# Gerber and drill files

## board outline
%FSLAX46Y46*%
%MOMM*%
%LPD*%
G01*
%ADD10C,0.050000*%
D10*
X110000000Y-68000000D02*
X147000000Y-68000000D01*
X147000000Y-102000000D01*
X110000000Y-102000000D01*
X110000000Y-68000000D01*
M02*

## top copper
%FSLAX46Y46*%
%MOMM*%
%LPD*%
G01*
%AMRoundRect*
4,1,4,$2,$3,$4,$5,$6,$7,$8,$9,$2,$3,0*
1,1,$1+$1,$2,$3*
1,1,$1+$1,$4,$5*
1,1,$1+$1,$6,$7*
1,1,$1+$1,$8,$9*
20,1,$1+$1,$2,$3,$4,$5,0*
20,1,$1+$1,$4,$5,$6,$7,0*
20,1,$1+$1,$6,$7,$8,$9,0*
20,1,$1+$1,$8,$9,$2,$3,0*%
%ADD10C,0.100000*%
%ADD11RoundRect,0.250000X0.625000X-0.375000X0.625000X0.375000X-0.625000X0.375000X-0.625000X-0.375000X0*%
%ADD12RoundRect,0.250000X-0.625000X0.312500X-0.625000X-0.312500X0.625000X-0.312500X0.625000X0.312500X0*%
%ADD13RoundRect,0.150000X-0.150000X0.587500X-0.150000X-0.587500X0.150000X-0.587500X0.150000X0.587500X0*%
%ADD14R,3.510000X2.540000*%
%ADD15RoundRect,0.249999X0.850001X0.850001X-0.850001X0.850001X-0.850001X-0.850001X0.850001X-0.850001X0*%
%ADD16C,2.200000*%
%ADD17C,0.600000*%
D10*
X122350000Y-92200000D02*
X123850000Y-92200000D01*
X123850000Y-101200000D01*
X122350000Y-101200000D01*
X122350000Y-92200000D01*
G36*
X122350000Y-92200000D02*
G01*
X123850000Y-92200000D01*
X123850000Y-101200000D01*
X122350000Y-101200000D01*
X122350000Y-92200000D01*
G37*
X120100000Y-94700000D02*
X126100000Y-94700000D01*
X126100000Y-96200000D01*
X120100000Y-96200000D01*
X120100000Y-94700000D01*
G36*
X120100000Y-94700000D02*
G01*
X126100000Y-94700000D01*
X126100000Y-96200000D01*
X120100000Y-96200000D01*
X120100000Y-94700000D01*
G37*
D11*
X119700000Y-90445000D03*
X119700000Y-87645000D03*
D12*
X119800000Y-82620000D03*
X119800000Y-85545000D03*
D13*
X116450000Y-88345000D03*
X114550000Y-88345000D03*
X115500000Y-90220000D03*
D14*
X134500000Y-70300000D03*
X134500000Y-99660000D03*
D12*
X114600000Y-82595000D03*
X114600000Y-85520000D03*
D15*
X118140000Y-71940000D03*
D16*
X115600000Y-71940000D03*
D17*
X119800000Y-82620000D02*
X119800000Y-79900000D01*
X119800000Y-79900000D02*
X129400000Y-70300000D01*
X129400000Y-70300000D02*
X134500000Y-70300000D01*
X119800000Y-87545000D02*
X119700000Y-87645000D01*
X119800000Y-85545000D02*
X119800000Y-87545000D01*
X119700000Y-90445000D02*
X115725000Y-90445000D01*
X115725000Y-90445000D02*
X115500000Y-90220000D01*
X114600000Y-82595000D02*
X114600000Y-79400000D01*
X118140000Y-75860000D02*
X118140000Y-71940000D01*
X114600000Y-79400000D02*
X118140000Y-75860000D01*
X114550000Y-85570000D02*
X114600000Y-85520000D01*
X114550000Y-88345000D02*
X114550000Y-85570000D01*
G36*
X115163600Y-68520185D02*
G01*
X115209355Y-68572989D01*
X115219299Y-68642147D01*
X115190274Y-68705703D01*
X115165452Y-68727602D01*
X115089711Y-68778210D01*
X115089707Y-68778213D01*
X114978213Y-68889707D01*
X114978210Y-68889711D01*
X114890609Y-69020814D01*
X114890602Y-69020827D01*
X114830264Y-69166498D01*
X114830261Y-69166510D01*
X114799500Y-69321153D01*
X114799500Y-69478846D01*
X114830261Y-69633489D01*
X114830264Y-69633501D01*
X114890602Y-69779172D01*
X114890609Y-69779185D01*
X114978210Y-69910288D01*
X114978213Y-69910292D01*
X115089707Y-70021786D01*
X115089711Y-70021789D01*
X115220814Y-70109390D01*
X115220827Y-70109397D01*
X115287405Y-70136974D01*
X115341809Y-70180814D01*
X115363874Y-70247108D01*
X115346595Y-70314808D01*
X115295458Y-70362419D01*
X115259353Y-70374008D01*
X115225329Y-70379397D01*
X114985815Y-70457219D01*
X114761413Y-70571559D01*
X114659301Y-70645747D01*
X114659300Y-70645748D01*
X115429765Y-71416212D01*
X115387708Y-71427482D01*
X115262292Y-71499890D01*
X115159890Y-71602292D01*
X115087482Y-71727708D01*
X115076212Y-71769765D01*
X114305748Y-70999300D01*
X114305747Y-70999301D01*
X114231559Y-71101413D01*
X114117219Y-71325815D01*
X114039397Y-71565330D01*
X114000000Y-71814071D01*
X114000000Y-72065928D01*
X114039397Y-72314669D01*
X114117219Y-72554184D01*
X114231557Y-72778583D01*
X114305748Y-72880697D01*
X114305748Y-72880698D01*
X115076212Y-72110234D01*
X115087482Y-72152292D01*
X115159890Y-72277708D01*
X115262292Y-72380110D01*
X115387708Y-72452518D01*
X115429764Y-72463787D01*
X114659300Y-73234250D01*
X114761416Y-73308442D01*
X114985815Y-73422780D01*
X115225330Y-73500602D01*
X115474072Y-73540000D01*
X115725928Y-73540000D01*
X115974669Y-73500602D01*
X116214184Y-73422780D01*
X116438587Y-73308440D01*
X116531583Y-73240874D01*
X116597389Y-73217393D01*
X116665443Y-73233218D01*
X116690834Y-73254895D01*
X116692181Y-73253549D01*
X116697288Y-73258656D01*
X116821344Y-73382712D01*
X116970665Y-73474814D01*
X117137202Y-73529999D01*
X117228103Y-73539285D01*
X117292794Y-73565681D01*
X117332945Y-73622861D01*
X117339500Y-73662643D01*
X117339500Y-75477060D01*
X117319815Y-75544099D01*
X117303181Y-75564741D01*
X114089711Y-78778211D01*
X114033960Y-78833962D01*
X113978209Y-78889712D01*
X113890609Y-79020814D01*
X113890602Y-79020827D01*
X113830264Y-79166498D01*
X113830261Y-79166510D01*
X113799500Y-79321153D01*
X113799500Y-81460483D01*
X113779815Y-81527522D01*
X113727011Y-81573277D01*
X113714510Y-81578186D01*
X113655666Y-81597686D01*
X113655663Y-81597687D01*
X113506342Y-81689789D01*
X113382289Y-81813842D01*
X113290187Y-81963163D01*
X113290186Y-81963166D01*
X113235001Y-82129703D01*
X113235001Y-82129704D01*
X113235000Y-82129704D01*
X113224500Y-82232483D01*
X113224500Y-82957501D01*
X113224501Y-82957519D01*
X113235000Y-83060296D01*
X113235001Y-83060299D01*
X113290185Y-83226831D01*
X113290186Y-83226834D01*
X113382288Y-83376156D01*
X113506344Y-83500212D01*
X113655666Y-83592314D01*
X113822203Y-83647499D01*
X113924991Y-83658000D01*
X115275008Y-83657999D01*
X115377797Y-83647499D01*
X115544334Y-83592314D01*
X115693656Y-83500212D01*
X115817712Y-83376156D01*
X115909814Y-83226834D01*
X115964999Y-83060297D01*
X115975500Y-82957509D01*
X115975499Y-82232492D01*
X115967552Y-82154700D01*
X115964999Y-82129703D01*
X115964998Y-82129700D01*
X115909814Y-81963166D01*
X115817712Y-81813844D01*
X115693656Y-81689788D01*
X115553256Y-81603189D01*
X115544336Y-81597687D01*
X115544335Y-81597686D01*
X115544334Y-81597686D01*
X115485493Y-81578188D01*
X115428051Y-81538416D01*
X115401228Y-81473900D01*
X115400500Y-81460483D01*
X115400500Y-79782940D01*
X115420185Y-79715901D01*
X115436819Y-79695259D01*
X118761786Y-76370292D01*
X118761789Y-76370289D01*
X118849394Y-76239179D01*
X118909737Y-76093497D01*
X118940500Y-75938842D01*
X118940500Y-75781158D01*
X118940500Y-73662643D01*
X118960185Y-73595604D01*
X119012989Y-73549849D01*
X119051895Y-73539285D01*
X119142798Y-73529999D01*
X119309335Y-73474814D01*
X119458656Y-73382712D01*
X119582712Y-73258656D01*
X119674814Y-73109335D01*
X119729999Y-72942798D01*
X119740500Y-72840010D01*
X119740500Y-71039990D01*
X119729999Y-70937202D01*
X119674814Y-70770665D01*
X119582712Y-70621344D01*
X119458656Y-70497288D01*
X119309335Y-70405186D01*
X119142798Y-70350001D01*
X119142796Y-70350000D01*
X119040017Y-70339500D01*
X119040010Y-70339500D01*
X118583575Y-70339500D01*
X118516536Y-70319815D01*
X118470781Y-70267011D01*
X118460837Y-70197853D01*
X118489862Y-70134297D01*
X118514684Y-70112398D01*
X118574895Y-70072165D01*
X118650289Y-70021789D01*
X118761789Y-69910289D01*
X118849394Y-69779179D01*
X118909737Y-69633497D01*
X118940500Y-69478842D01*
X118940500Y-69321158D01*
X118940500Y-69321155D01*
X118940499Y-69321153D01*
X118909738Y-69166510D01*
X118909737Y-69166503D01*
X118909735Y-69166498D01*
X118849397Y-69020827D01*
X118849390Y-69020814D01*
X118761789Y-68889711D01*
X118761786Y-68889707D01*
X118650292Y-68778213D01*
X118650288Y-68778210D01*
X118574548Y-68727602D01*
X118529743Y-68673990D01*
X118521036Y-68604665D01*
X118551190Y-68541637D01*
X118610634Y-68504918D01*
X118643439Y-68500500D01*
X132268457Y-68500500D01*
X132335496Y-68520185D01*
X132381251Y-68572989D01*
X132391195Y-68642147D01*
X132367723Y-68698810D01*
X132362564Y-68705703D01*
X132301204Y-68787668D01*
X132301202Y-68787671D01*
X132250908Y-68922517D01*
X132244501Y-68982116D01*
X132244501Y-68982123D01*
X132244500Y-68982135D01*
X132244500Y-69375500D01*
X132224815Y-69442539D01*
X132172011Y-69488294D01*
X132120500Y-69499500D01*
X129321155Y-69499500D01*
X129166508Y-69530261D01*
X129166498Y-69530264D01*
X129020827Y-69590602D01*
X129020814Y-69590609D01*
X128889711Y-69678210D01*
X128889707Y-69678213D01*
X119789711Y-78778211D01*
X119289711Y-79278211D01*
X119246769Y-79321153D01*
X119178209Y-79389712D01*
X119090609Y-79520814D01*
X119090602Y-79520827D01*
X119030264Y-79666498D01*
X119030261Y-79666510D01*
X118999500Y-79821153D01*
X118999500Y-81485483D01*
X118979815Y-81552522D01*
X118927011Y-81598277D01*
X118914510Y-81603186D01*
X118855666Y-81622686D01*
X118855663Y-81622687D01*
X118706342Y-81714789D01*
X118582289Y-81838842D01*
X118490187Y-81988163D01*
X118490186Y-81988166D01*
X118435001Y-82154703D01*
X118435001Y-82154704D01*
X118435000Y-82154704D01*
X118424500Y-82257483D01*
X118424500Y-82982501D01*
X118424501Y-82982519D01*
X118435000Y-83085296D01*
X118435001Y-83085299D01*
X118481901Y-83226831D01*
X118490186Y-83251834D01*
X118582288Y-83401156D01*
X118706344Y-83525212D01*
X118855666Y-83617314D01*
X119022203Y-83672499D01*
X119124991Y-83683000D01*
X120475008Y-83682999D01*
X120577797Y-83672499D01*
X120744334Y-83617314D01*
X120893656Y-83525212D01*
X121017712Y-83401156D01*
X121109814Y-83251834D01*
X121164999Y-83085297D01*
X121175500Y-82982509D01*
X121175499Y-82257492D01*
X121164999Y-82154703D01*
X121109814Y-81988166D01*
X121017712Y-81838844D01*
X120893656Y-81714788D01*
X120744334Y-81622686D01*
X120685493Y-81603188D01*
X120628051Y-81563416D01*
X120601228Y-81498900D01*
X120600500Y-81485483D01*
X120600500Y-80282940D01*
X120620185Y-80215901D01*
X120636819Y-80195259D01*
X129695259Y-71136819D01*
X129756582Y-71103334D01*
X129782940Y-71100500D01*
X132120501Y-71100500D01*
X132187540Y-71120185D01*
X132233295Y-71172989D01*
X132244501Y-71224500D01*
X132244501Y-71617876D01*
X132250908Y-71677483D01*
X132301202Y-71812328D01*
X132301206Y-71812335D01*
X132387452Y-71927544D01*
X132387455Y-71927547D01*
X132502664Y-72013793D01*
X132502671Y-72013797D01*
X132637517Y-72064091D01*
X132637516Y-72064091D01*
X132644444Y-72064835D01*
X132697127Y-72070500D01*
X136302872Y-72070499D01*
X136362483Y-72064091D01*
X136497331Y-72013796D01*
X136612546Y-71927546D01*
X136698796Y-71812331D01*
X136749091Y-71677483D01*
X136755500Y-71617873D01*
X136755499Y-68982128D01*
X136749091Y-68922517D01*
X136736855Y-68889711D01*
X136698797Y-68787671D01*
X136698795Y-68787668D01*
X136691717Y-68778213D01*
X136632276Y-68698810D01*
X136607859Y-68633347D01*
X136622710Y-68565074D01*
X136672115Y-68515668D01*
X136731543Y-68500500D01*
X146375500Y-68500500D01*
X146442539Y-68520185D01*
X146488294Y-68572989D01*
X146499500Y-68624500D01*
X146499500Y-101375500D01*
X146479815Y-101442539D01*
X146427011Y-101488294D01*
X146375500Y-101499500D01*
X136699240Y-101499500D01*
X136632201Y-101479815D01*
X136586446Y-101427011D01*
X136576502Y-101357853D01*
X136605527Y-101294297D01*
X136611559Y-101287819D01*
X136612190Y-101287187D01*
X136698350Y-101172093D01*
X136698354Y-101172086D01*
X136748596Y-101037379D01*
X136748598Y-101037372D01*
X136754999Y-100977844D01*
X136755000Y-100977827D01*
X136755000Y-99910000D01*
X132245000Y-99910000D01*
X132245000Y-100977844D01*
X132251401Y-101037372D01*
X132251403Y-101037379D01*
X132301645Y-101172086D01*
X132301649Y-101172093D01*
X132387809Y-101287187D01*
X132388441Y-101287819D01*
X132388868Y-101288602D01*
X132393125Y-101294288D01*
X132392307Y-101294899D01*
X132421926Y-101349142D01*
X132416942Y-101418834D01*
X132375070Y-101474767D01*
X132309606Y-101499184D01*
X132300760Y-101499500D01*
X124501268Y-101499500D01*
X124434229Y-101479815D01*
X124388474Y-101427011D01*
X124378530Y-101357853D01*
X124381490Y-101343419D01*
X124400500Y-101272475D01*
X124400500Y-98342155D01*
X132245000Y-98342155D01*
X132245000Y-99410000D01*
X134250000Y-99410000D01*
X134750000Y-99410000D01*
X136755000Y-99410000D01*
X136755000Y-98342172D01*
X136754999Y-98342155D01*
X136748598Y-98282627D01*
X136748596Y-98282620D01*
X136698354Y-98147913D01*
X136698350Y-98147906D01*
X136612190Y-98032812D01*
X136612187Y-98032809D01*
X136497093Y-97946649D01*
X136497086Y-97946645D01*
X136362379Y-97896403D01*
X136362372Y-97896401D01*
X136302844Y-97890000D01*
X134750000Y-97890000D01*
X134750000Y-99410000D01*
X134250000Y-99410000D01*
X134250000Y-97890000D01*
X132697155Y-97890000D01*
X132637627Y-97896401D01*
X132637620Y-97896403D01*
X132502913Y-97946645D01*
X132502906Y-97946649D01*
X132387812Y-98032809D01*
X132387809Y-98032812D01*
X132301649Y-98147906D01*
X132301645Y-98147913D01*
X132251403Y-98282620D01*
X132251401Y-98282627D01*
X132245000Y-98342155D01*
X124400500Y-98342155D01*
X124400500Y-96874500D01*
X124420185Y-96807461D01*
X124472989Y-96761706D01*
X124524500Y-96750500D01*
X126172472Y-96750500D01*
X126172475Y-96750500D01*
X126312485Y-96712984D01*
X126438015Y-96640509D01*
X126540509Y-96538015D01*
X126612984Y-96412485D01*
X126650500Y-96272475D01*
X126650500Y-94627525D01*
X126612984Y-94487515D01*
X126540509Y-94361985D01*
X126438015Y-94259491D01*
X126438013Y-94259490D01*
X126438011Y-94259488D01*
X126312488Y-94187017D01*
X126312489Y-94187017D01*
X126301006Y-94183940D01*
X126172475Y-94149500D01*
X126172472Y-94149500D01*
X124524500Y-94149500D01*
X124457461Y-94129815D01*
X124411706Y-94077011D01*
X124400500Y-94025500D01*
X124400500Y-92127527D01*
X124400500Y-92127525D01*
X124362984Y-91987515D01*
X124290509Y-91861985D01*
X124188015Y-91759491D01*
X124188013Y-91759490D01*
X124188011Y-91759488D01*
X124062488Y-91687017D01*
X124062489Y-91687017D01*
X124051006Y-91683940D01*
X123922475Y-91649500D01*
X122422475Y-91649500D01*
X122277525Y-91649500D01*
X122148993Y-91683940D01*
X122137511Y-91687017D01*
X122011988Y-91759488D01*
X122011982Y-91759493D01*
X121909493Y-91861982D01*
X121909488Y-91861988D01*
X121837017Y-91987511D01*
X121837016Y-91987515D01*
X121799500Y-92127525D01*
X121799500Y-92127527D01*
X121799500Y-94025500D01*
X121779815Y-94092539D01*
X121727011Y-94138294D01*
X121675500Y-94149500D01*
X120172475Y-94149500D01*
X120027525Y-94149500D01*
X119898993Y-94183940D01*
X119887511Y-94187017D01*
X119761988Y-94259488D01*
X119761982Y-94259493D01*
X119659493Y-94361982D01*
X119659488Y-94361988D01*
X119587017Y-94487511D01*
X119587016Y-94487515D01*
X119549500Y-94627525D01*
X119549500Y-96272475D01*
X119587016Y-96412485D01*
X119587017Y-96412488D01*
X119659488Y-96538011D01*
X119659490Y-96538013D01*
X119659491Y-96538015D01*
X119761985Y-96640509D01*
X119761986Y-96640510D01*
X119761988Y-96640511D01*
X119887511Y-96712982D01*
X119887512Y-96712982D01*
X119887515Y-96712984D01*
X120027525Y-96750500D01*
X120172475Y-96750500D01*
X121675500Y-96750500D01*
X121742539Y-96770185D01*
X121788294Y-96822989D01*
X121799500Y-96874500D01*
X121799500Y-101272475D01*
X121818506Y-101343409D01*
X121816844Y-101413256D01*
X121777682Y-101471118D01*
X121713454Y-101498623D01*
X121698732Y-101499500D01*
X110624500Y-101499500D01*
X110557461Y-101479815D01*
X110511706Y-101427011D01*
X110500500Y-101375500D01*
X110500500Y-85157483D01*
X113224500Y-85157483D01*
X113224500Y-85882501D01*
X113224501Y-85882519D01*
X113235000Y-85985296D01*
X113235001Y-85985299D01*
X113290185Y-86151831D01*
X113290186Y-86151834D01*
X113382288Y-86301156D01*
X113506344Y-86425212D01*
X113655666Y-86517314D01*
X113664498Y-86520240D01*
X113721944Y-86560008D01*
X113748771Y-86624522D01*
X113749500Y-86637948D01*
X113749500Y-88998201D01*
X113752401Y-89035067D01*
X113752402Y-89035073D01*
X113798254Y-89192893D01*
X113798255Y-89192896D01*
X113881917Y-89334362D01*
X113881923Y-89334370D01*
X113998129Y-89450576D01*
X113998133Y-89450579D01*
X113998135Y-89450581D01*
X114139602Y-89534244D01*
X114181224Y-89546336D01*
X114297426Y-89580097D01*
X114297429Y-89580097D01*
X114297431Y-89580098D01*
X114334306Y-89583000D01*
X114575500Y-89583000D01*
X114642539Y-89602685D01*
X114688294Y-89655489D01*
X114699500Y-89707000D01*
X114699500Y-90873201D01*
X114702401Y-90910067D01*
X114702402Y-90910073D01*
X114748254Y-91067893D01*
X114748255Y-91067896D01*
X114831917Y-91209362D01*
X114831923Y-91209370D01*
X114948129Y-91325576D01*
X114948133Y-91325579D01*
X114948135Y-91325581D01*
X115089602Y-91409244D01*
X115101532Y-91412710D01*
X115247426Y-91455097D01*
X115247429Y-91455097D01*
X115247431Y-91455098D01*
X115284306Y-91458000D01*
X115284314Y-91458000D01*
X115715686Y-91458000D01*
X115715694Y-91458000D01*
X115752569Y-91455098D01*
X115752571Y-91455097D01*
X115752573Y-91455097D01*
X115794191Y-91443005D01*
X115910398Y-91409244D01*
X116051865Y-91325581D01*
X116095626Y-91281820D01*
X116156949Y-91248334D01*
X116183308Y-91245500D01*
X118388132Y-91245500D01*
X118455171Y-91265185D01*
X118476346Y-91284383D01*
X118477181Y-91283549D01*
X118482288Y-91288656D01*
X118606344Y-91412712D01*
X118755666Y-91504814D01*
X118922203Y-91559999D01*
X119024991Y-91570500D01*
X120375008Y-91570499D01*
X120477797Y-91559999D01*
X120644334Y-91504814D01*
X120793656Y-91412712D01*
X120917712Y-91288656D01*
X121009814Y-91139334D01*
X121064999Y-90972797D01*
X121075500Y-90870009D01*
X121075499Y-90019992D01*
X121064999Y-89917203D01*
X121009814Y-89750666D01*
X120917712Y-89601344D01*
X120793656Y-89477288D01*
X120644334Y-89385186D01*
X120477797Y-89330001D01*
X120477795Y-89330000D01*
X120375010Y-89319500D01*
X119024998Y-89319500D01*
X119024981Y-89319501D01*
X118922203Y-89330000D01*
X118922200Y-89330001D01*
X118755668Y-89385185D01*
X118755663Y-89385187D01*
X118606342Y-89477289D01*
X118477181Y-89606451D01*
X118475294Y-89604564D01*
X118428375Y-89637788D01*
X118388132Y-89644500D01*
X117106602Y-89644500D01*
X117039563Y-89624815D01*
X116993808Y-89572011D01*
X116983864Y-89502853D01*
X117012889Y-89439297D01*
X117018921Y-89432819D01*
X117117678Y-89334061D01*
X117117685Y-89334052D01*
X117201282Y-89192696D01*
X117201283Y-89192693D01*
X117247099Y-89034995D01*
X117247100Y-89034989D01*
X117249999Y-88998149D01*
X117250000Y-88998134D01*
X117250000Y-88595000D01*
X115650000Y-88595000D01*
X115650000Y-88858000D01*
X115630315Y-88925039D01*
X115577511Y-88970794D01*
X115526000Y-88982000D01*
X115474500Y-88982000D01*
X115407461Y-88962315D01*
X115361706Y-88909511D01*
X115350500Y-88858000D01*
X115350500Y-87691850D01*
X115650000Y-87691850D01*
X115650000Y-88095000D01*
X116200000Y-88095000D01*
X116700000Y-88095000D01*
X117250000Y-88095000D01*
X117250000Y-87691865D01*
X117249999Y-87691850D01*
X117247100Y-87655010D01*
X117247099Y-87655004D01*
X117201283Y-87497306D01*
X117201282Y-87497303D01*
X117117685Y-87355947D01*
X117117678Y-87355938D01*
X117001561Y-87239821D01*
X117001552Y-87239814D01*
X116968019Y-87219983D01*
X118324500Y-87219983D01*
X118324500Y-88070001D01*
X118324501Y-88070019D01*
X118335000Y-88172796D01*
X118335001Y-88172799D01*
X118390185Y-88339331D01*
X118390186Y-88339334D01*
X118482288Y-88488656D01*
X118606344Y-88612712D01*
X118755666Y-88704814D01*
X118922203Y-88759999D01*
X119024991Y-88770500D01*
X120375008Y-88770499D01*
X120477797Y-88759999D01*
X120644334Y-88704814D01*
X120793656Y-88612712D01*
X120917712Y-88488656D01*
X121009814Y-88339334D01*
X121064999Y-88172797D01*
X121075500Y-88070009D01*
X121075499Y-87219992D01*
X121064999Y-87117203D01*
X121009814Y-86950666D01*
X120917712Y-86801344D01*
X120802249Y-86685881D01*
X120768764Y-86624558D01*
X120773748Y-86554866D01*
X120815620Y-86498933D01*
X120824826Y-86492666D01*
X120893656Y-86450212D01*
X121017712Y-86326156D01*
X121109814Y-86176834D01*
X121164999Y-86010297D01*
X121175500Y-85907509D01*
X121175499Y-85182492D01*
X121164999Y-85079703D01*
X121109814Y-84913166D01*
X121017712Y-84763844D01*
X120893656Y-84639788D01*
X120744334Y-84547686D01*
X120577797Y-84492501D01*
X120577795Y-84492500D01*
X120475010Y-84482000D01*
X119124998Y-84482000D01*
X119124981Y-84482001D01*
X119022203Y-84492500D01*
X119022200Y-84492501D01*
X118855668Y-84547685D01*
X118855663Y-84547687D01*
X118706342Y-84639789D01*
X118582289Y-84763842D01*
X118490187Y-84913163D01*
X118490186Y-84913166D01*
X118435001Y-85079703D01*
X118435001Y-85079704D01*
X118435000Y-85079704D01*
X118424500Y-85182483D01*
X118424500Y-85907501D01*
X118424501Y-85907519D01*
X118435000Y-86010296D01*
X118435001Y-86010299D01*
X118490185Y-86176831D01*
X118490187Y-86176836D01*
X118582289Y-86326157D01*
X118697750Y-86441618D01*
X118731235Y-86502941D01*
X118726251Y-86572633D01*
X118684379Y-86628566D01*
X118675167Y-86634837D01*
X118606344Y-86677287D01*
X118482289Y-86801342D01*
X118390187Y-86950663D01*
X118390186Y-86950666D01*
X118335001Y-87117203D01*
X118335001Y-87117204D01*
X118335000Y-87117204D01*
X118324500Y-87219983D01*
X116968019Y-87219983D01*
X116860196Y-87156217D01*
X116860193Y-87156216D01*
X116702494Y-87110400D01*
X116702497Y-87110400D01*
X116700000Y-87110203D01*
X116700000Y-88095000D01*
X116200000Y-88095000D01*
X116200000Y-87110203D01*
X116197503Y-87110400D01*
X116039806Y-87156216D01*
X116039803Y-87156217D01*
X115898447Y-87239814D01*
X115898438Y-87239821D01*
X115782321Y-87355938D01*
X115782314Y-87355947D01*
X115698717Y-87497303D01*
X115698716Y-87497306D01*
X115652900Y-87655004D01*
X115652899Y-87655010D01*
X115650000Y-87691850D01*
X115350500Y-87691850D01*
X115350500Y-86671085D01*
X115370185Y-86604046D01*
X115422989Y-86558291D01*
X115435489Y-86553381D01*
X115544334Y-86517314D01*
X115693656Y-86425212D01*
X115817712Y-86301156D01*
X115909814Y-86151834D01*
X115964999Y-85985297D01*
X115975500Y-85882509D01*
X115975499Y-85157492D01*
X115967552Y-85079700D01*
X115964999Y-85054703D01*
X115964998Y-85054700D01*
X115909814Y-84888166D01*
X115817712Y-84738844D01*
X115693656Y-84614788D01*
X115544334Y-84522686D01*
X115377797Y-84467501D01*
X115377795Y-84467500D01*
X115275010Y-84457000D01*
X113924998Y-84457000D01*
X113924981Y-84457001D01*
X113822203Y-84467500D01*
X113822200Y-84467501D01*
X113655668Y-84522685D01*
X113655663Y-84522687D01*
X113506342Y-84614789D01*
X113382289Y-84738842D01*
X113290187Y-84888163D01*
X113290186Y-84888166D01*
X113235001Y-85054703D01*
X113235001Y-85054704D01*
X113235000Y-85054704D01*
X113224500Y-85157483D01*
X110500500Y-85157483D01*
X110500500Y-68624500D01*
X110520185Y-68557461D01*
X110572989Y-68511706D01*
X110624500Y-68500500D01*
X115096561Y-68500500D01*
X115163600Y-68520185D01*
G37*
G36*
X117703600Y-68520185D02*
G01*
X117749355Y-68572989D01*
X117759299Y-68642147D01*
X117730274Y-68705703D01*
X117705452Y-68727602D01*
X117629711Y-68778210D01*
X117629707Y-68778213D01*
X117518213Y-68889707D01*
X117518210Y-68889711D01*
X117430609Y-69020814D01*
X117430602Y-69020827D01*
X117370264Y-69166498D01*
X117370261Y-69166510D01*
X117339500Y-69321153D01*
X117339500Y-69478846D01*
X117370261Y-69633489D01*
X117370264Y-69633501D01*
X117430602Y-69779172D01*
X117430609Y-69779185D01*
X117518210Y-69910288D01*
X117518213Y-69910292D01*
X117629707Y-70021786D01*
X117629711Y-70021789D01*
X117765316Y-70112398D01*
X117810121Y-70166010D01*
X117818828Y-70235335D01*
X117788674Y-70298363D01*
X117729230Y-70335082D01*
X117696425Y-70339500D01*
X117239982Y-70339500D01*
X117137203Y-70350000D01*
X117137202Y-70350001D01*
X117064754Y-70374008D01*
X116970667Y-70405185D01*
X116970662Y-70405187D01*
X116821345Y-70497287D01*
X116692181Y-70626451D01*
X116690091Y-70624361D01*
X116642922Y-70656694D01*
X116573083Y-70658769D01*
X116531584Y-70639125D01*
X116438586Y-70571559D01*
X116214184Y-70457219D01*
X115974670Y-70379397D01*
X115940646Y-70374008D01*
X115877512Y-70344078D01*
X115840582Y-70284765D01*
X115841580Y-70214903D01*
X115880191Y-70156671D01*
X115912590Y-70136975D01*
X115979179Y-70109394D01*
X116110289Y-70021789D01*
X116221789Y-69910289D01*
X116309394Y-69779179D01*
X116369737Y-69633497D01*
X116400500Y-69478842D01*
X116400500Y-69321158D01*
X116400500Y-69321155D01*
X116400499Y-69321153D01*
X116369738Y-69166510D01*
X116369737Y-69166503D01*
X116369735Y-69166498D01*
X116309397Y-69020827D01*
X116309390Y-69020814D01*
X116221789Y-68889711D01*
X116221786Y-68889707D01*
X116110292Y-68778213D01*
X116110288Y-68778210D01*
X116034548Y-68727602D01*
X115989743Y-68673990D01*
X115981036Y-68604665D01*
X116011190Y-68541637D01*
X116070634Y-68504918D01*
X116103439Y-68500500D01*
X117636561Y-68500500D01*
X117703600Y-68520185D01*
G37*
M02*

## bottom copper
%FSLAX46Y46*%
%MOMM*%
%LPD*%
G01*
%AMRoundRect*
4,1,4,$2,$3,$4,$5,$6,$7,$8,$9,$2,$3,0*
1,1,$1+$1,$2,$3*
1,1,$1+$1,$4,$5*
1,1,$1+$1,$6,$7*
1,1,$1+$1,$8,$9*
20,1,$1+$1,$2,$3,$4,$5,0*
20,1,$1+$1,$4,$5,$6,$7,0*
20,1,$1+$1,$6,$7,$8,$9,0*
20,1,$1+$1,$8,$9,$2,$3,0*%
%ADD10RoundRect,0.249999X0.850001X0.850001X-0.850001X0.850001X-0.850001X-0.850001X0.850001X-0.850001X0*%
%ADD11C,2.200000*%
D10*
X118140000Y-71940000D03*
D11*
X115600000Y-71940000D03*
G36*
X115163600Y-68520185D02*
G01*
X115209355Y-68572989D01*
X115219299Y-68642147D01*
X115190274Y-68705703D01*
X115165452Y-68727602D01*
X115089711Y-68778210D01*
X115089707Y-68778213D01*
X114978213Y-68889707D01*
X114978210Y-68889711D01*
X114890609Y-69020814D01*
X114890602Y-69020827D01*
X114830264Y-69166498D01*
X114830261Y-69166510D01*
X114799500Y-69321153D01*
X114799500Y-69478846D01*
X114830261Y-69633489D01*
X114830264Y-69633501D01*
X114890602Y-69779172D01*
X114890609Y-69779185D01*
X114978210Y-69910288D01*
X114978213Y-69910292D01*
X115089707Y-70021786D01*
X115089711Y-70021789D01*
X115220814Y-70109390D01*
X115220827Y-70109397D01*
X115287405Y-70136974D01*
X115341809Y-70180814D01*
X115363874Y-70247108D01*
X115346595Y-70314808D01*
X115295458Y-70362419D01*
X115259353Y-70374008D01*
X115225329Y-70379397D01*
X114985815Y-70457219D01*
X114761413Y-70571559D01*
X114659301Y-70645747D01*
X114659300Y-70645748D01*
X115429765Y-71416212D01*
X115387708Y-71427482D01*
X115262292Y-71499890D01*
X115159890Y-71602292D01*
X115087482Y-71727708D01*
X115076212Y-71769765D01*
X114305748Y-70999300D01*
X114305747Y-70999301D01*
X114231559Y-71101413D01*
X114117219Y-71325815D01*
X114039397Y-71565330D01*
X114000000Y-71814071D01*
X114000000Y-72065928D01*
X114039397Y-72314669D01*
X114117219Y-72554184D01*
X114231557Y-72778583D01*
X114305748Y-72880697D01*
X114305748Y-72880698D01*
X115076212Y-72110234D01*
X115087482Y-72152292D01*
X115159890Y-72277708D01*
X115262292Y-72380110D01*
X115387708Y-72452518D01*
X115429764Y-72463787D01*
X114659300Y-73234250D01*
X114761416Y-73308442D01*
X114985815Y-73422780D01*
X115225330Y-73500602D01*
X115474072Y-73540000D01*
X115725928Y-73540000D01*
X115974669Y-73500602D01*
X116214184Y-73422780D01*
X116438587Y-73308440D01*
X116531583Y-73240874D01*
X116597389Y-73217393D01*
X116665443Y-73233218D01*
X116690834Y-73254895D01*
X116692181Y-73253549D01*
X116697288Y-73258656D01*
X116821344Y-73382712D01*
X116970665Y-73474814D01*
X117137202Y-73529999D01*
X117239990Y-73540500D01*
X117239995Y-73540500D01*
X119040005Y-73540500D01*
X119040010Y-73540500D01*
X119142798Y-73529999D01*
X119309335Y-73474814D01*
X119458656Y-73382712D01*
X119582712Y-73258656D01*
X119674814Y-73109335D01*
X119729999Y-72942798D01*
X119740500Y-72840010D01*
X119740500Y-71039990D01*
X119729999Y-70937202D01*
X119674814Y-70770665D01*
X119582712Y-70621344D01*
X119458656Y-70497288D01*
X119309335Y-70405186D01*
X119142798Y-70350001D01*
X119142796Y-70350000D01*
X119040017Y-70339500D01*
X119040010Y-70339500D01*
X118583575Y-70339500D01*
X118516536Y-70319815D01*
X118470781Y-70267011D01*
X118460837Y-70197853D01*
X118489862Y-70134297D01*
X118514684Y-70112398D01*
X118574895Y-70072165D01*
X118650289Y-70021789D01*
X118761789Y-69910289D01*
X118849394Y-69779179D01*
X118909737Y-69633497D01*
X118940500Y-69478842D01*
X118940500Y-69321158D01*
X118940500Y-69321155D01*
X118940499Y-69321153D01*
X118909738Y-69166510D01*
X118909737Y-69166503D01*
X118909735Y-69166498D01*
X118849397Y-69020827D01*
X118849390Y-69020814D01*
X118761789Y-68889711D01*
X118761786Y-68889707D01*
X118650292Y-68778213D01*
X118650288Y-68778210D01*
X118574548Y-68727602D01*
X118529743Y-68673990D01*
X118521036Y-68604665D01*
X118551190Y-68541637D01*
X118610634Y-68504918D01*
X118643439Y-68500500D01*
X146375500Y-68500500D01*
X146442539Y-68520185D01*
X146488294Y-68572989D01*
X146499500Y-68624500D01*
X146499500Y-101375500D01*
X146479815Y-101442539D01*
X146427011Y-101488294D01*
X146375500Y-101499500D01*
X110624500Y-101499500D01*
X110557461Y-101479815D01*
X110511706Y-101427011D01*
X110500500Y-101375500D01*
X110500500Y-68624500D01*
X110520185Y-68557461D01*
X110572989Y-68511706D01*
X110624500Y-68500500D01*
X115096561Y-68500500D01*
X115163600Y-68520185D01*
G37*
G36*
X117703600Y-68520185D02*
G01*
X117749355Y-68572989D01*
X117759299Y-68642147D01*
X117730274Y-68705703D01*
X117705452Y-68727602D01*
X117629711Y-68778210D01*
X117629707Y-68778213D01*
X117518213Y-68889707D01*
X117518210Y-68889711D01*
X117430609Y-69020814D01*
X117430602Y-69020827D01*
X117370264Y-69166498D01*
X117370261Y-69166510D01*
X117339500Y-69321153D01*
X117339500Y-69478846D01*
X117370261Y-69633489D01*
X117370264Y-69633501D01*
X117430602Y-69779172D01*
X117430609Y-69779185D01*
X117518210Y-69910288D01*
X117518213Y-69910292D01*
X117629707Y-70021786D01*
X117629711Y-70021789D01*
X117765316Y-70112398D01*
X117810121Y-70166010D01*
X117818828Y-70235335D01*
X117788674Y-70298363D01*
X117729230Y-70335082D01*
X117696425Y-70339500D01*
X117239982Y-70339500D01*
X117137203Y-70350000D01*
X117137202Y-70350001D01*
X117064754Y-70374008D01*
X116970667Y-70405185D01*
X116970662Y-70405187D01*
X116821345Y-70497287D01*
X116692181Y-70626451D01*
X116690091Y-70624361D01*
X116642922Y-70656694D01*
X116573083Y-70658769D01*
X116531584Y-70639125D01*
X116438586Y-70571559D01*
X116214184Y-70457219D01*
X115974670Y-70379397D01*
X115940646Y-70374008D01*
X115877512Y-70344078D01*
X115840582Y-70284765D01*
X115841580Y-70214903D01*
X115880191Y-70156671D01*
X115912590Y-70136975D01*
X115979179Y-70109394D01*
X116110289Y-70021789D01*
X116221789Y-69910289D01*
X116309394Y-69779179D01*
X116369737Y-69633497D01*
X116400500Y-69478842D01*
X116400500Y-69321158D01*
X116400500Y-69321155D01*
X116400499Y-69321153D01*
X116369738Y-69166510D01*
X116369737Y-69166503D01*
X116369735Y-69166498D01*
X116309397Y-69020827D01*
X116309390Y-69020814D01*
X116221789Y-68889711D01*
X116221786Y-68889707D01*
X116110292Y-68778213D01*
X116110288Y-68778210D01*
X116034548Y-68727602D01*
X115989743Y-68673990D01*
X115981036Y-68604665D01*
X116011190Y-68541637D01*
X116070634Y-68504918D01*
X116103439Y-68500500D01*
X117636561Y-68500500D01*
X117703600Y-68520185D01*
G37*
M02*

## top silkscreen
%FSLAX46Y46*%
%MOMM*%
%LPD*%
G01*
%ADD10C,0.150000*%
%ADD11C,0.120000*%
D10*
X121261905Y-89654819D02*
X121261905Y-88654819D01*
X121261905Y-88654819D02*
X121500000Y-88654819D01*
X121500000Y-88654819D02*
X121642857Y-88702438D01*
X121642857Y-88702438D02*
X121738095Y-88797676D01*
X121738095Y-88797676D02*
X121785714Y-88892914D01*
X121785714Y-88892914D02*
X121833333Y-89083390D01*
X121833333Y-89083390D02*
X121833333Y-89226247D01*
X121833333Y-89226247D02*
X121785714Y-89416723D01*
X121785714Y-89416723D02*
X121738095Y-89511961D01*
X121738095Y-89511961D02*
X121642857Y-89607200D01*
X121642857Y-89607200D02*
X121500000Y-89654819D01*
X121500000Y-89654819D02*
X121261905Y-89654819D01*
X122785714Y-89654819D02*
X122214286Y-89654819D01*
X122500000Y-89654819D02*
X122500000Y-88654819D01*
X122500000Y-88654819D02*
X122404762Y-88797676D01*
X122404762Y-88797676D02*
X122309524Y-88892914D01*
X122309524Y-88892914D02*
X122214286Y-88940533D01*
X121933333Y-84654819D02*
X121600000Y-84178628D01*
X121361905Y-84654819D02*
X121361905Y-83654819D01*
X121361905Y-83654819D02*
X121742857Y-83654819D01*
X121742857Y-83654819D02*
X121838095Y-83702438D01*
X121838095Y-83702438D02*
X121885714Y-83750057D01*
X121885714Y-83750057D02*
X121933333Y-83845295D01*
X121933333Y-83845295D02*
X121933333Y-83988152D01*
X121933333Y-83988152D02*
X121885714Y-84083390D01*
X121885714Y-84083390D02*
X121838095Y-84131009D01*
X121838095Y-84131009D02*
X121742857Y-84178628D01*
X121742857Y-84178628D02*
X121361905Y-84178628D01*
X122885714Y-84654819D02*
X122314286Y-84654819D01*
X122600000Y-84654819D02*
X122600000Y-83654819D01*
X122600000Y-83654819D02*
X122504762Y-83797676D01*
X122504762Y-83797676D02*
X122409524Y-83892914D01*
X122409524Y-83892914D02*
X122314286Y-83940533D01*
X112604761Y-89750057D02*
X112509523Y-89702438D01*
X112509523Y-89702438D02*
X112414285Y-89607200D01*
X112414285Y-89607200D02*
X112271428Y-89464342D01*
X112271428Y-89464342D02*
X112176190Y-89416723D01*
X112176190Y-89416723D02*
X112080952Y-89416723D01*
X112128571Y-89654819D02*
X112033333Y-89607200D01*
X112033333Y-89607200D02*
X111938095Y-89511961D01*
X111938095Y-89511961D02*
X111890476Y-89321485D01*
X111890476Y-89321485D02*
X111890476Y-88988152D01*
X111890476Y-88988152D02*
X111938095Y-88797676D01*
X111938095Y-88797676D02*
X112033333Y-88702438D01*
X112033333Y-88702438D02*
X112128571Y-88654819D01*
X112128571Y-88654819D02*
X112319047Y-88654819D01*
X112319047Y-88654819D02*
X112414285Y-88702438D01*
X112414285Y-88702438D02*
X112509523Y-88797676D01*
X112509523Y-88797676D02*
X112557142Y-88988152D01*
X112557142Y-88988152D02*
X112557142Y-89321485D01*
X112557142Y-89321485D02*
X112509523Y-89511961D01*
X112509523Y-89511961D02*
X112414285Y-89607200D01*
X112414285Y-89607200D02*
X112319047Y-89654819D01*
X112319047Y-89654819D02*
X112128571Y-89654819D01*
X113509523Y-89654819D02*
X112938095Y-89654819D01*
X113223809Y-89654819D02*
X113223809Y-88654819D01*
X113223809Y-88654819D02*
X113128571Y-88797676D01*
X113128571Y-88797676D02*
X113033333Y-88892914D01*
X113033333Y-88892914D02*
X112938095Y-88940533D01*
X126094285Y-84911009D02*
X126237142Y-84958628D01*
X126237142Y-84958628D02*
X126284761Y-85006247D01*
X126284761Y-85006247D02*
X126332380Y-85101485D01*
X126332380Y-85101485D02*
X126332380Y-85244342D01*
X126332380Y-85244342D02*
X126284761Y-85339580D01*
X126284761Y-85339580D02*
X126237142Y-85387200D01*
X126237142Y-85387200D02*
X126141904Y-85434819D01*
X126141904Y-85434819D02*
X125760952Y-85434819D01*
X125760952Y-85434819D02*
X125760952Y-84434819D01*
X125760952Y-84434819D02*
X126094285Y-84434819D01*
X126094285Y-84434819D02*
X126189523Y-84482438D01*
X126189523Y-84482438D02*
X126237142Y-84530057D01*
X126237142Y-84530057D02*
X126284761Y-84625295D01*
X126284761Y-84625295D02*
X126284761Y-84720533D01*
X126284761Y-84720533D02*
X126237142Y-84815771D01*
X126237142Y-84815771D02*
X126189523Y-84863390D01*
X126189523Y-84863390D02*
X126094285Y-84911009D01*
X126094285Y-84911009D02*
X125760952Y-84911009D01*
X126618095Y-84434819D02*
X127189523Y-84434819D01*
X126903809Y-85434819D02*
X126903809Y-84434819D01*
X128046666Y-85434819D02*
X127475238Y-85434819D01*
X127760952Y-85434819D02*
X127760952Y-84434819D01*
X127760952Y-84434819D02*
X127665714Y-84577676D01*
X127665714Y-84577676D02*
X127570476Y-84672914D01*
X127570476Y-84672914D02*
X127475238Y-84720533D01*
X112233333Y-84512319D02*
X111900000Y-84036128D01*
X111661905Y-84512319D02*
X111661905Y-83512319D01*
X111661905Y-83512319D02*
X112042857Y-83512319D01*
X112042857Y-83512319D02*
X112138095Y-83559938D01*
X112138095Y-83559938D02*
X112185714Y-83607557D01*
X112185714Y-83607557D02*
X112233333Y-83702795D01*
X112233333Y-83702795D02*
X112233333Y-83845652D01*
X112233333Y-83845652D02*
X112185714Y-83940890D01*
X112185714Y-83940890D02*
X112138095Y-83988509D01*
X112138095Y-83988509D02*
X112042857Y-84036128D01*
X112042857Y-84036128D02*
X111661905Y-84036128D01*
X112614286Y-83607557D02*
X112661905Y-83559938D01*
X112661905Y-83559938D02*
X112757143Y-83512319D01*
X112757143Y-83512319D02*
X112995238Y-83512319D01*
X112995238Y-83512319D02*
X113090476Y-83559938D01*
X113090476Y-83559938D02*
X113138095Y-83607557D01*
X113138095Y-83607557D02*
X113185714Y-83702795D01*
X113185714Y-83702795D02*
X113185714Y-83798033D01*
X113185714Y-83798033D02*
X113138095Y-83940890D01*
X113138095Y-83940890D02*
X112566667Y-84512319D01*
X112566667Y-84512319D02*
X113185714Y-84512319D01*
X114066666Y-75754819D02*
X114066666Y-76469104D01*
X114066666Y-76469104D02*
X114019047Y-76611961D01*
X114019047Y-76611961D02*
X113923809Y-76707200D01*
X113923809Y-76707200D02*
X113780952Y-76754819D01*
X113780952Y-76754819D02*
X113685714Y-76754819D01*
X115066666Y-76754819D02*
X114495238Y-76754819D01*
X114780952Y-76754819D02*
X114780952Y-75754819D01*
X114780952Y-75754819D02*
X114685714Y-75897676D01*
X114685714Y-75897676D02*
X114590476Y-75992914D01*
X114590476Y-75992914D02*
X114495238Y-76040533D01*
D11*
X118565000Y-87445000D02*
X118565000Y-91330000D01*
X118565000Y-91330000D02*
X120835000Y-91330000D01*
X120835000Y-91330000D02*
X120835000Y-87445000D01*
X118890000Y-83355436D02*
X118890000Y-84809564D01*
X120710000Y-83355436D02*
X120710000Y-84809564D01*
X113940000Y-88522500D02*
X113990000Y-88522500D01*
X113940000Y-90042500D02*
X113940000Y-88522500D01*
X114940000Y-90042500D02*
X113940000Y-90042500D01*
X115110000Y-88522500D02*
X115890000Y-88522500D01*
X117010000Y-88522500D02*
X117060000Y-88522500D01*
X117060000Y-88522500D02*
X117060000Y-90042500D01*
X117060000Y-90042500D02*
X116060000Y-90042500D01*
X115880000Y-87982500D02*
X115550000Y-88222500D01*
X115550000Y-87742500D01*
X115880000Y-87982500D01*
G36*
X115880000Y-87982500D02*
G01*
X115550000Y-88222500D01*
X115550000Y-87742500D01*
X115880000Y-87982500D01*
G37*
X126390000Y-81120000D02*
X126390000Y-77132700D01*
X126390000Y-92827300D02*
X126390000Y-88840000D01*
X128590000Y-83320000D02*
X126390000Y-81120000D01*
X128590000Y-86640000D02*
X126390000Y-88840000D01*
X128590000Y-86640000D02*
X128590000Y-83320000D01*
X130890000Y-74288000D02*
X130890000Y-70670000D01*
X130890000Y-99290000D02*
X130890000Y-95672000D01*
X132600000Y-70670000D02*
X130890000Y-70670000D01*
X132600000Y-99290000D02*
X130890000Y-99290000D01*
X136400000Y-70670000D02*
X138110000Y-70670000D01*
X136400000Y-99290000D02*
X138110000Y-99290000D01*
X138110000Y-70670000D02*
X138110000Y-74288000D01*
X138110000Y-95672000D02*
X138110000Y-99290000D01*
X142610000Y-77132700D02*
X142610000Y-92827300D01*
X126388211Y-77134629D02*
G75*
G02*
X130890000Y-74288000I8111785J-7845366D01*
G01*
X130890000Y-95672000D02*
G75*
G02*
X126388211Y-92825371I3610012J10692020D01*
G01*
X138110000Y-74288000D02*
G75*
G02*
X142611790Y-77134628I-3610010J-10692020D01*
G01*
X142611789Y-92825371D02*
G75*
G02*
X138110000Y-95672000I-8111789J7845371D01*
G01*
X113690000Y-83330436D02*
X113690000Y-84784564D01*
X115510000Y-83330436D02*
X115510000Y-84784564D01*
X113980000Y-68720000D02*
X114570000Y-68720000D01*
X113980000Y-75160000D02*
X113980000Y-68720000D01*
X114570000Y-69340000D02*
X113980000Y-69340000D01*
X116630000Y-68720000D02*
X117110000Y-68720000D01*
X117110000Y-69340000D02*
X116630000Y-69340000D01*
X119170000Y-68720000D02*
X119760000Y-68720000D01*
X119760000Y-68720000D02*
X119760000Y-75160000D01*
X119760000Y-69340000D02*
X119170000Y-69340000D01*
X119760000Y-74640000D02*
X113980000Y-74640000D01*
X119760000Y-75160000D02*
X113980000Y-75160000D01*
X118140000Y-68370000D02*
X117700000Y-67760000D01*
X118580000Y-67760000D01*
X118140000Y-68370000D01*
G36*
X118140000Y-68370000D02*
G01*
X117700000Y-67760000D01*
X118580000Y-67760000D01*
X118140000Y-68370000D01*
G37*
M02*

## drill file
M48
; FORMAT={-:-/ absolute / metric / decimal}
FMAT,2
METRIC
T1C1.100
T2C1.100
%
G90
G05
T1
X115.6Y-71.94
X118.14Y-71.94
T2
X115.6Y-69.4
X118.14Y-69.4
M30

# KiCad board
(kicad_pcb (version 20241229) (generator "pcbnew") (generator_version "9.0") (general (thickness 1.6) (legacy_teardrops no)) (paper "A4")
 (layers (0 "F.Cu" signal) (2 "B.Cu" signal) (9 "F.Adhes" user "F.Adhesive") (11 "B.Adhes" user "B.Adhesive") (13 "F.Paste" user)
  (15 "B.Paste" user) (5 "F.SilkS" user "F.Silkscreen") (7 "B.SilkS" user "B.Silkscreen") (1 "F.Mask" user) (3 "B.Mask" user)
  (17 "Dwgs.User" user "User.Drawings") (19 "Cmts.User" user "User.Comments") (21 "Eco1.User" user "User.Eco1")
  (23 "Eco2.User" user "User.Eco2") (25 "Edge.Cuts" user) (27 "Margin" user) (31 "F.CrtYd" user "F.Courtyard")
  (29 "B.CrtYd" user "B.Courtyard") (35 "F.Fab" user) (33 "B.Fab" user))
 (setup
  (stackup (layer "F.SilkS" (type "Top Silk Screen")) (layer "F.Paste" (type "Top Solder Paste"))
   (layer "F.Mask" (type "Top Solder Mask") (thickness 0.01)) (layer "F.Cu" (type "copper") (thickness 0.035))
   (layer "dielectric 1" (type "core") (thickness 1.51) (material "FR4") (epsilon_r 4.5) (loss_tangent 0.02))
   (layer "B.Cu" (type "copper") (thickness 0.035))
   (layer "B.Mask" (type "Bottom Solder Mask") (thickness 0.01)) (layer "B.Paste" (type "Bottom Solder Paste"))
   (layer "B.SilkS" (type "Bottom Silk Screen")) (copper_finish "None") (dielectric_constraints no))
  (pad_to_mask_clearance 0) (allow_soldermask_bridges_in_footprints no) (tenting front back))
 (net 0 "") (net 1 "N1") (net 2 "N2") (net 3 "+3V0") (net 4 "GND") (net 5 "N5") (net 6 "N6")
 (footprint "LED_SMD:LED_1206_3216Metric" (layer "F.Cu") (at 119.7 89.045 90)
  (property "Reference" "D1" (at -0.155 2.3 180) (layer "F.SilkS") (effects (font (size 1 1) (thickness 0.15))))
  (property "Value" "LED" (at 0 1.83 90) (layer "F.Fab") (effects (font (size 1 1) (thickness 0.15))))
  (fp_line (start 1.6 -1.135) (end -2.285 -1.135) (stroke (width 0.12) (type solid)) (layer "F.SilkS"))
  (fp_line (start -2.285 -1.135) (end -2.285 1.135) (stroke (width 0.12) (type solid)) (layer "F.SilkS"))
  (fp_line (start -2.285 1.135) (end 1.6 1.135) (stroke (width 0.12) (type solid)) (layer "F.SilkS"))
  (pad "1" smd roundrect (at -1.4 0 90) (size 1.25 1.75) (layers "F.Cu" "F.Mask" "F.Paste") (roundrect_rratio 0.2) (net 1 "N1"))
  (pad "2" smd roundrect (at 1.4 0 90) (size 1.25 1.75) (layers "F.Cu" "F.Mask" "F.Paste") (roundrect_rratio 0.2) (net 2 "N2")))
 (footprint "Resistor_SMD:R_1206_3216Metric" (layer "F.Cu") (at 119.8 84.0825 -90)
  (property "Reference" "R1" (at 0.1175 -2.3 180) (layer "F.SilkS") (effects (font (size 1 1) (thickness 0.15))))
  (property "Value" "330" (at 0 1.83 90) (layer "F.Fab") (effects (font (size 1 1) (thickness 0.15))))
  (fp_line (start -0.727064 0.91) (end 0.727064 0.91) (stroke (width 0.12) (type solid)) (layer "F.SilkS"))
  (fp_line (start -0.727064 -0.91) (end 0.727064 -0.91) (stroke (width 0.12) (type solid)) (layer "F.SilkS"))
  (pad "1" smd roundrect (at -1.4625 0 270) (size 1.125 1.75) (layers "F.Cu" "F.Mask" "F.Paste") (roundrect_rratio 0.222222) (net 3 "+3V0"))
  (pad "2" smd roundrect (at 1.4625 0 270) (size 1.125 1.75) (layers "F.Cu" "F.Mask" "F.Paste") (roundrect_rratio 0.222222) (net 2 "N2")))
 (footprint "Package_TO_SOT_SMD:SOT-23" (layer "F.Cu") (at 115.5 89.2825 -90)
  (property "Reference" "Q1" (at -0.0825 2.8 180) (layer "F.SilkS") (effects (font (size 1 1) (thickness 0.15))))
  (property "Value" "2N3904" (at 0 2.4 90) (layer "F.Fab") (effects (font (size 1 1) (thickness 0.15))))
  (fp_line (start -0.76 1.56) (end -0.76 1.51) (stroke (width 0.12) (type solid)) (layer "F.SilkS"))
  (fp_line (start 0.76 1.56) (end -0.76 1.56) (stroke (width 0.12) (type solid)) (layer "F.SilkS"))
  (fp_line (start 0.76 0.56) (end 0.76 1.56) (stroke (width 0.12) (type solid)) (layer "F.SilkS"))
  (fp_line (start -0.76 0.39) (end -0.76 -0.39) (stroke (width 0.12) (type solid)) (layer "F.SilkS"))
  (fp_line (start -0.76 -1.51) (end -0.76 -1.56) (stroke (width 0.12) (type solid)) (layer "F.SilkS"))
  (fp_line (start -0.76 -1.56) (end 0.76 -1.56) (stroke (width 0.12) (type solid)) (layer "F.SilkS"))
  (fp_line (start 0.76 -1.56) (end 0.76 -0.56) (stroke (width 0.12) (type solid)) (layer "F.SilkS"))
  (fp_poly (pts (xy -1.3 -0.38) (xy -1.06 -0.05) (xy -1.54 -0.05)) (stroke (width 0.12) (type solid)) (fill yes) (layer "F.SilkS"))
  (pad "1" smd roundrect (at -0.9375 -0.95 270) (size 1.475 0.6) (layers "F.Cu" "F.Mask" "F.Paste") (roundrect_rratio 0.25) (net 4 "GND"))
  (pad "2" smd roundrect (at -0.9375 0.95 270) (size 1.475 0.6) (layers "F.Cu" "F.Mask" "F.Paste") (roundrect_rratio 0.25) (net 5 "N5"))
  (pad "3" smd roundrect (at 0.9375 0 270) (size 1.475 0.6) (layers "F.Cu" "F.Mask" "F.Paste") (roundrect_rratio 0.25) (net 1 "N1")))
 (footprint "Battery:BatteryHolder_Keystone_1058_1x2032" (layer "F.Cu") (at 134.5 84.98 -90)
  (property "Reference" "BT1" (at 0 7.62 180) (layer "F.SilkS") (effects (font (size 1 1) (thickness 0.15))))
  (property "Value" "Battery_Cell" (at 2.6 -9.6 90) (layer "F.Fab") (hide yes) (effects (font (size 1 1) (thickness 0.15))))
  (fp_line (start -3.86 8.11) (end -7.8473 8.11) (stroke (width 0.12) (type solid)) (layer "F.SilkS"))
  (fp_line (start 7.8473 8.11) (end 3.86 8.11) (stroke (width 0.12) (type solid)) (layer "F.SilkS"))
  (fp_line (start -1.66 5.91) (end -3.86 8.11) (stroke (width 0.12) (type solid)) (layer "F.SilkS"))
  (fp_line (start 1.66 5.91) (end 3.86 8.11) (stroke (width 0.12) (type solid)) (layer "F.SilkS"))
  (fp_line (start 1.66 5.91) (end -1.66 5.91) (stroke (width 0.12) (type solid)) (layer "F.SilkS"))
  (fp_line (start -10.692 3.61) (end -14.31 3.61) (stroke (width 0.12) (type solid)) (layer "F.SilkS"))
  (fp_line (start 14.31 3.61) (end 10.692 3.61) (stroke (width 0.12) (type solid)) (layer "F.SilkS"))
  (fp_line (start -14.31 1.9) (end -14.31 3.61) (stroke (width 0.12) (type solid)) (layer "F.SilkS"))
  (fp_line (start 14.31 1.9) (end 14.31 3.61) (stroke (width 0.12) (type solid)) (layer "F.SilkS"))
  (fp_line (start -14.31 -1.9) (end -14.31 -3.61) (stroke (width 0.12) (type solid)) (layer "F.SilkS"))
  (fp_line (start 14.31 -1.9) (end 14.31 -3.61) (stroke (width 0.12) (type solid)) (layer "F.SilkS"))
  (fp_line (start -14.31 -3.61) (end -10.692 -3.61) (stroke (width 0.12) (type solid)) (layer "F.SilkS"))
  (fp_line (start 10.692 -3.61) (end 14.31 -3.61) (stroke (width 0.12) (type solid)) (layer "F.SilkS"))
  (fp_line (start -7.8473 -8.11) (end 7.8473 -8.11) (stroke (width 0.12) (type solid)) (layer "F.SilkS"))
  (fp_arc (start -7.845371 8.111789) (mid -9.538085 6.031244) (end -10.692 3.61) (stroke (width 0.12) (type solid)) (layer "F.SilkS"))
  (fp_arc (start 10.692 3.61) (mid 9.538084 6.031244) (end 7.845371 8.111789) (stroke (width 0.12) (type solid)) (layer "F.SilkS"))
  (fp_arc (start -10.692 -3.61) (mid -9.538084 -6.031244) (end -7.845371 -8.111789) (stroke (width 0.12) (type solid)) (layer "F.SilkS"))
  (fp_arc (start 7.845371 -8.111789) (mid 9.538085 -6.031244) (end 10.692 -3.61) (stroke (width 0.12) (type solid)) (layer "F.SilkS"))
  (pad "1" smd rect (at -14.68 0 270) (size 2.54 3.51) (layers "F.Cu" "F.Mask" "F.Paste") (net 3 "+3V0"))
  (pad "2" smd rect (at 14.68 0 270) (size 2.54 3.51) (layers "F.Cu" "F.Mask" "F.Paste") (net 4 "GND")))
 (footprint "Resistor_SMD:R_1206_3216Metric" (layer "F.Cu") (at 114.6 84.0575 -90)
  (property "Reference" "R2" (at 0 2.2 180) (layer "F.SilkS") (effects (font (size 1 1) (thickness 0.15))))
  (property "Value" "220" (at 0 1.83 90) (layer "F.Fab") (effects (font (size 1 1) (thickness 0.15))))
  (fp_line (start -0.727064 0.91) (end 0.727064 0.91) (stroke (width 0.12) (type solid)) (layer "F.SilkS"))
  (fp_line (start -0.727064 -0.91) (end 0.727064 -0.91) (stroke (width 0.12) (type solid)) (layer "F.SilkS"))
  (pad "1" smd roundrect (at -1.4625 0 270) (size 1.125 1.75) (layers "F.Cu" "F.Mask" "F.Paste") (roundrect_rratio 0.222222) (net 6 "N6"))
  (pad "2" smd roundrect (at 1.4625 0 270) (size 1.125 1.75) (layers "F.Cu" "F.Mask" "F.Paste") (roundrect_rratio 0.222222) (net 5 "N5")))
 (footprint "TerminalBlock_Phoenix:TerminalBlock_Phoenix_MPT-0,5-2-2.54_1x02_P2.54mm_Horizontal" (layer "F.Cu") (at 118.14 71.94 180)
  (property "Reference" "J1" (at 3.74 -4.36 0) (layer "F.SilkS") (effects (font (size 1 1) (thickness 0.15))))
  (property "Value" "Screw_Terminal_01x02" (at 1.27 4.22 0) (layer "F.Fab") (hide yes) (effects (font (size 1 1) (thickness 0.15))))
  (fp_line (start 4.16 3.22) (end 3.57 3.22) (stroke (width 0.12) (type solid)) (layer "F.SilkS"))
  (fp_line (start 4.16 -3.22) (end 4.16 3.22) (stroke (width 0.12) (type solid)) (layer "F.SilkS"))
  (fp_line (start 3.57 2.6) (end 4.16 2.6) (stroke (width 0.12) (type solid)) (layer "F.SilkS"))
  (fp_line (start 1.51 3.22) (end 1.03 3.22) (stroke (width 0.12) (type solid)) (layer "F.SilkS"))
  (fp_line (start 1.03 2.6) (end 1.51 2.6) (stroke (width 0.12) (type solid)) (layer "F.SilkS"))
  (fp_line (start -1.03 3.22) (end -1.62 3.22) (stroke (width 0.12) (type solid)) (layer "F.SilkS"))
  (fp_line (start -1.62 3.22) (end -1.62 -3.22) (stroke (width 0.12) (type solid)) (layer "F.SilkS"))
  (fp_line (start -1.62 2.6) (end -1.03 2.6) (stroke (width 0.12) (type solid)) (layer "F.SilkS"))
  (fp_line (start -1.62 -2.7) (end 4.16 -2.7) (stroke (width 0.12) (type solid)) (layer "F.SilkS"))
  (fp_line (start -1.62 -3.22) (end 4.16 -3.22) (stroke (width 0.12) (type solid)) (layer "F.SilkS"))
  (fp_poly (pts (xy 0 3.57) (xy 0.44 4.18) (xy -0.44 4.18)) (stroke (width 0.12) (type solid)) (fill yes) (layer "F.SilkS"))
  (pad "" np_thru_hole circle (at 0 2.54 180) (size 1.1 1.1) (drill 1.1) (layers "*.Cu" "*.Mask"))
  (pad "" np_thru_hole circle (at 2.54 2.54 180) (size 1.1 1.1) (drill 1.1) (layers "*.Cu" "*.Mask"))
  (pad "1" thru_hole roundrect (at 0 0 180) (size 2.2 2.2) (drill 1.1) (layers "*.Cu" "*.Mask") (remove_unused_layers no)
   (roundrect_rratio 0.113636) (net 6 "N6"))
  (pad "2" thru_hole circle (at 2.54 0 180) (size 2.2 2.2) (drill 1.1) (layers "*.Cu" "*.Mask") (remove_unused_layers no) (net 4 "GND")))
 (gr_rect (start 122.35 92.2) (end 123.85 101.2) (stroke (width 0.1) (type solid)) (fill yes) (layer "F.Cu"))
 (gr_rect (start 120.1 94.7) (end 126.1 96.2) (stroke (width 0.1) (type solid)) (fill yes) (layer "F.Cu"))
 (gr_rect (start 110 68) (end 147 102) (stroke (width 0.05) (type default)) (fill no) (layer "Edge.Cuts"))
 (segment (start 119.8 82.62) (end 119.8 79.9) (width 0.6) (layer "F.Cu") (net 3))
 (segment (start 119.8 79.9) (end 129.4 70.3) (width 0.6) (layer "F.Cu") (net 3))
 (segment (start 129.4 70.3) (end 134.5 70.3) (width 0.6) (layer "F.Cu") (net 3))
 (segment (start 119.8 87.545) (end 119.7 87.645) (width 0.6) (layer "F.Cu") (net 2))
 (segment (start 119.8 85.545) (end 119.8 87.545) (width 0.6) (layer "F.Cu") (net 2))
 (segment (start 119.7 90.445) (end 115.725 90.445) (width 0.6) (layer "F.Cu") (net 1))
 (segment (start 115.725 90.445) (end 115.5 90.22) (width 0.6) (layer "F.Cu") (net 1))
 (segment (start 114.6 82.595) (end 114.6 79.4) (width 0.6) (layer "F.Cu") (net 6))
 (segment (start 118.14 75.86) (end 118.14 71.94) (width 0.6) (layer "F.Cu") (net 6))
 (segment (start 114.6 79.4) (end 118.14 75.86) (width 0.6) (layer "F.Cu") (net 6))
 (segment (start 114.55 85.57) (end 114.6 85.52) (width 0.6) (layer "F.Cu") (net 5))
 (segment (start 114.55 88.345) (end 114.55 85.57) (width 0.6) (layer "F.Cu") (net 5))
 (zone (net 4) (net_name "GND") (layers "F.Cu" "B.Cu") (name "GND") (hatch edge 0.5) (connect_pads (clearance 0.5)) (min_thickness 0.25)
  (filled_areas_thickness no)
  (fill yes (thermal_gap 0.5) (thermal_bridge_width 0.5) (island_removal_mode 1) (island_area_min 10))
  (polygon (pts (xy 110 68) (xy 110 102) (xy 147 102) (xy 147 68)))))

